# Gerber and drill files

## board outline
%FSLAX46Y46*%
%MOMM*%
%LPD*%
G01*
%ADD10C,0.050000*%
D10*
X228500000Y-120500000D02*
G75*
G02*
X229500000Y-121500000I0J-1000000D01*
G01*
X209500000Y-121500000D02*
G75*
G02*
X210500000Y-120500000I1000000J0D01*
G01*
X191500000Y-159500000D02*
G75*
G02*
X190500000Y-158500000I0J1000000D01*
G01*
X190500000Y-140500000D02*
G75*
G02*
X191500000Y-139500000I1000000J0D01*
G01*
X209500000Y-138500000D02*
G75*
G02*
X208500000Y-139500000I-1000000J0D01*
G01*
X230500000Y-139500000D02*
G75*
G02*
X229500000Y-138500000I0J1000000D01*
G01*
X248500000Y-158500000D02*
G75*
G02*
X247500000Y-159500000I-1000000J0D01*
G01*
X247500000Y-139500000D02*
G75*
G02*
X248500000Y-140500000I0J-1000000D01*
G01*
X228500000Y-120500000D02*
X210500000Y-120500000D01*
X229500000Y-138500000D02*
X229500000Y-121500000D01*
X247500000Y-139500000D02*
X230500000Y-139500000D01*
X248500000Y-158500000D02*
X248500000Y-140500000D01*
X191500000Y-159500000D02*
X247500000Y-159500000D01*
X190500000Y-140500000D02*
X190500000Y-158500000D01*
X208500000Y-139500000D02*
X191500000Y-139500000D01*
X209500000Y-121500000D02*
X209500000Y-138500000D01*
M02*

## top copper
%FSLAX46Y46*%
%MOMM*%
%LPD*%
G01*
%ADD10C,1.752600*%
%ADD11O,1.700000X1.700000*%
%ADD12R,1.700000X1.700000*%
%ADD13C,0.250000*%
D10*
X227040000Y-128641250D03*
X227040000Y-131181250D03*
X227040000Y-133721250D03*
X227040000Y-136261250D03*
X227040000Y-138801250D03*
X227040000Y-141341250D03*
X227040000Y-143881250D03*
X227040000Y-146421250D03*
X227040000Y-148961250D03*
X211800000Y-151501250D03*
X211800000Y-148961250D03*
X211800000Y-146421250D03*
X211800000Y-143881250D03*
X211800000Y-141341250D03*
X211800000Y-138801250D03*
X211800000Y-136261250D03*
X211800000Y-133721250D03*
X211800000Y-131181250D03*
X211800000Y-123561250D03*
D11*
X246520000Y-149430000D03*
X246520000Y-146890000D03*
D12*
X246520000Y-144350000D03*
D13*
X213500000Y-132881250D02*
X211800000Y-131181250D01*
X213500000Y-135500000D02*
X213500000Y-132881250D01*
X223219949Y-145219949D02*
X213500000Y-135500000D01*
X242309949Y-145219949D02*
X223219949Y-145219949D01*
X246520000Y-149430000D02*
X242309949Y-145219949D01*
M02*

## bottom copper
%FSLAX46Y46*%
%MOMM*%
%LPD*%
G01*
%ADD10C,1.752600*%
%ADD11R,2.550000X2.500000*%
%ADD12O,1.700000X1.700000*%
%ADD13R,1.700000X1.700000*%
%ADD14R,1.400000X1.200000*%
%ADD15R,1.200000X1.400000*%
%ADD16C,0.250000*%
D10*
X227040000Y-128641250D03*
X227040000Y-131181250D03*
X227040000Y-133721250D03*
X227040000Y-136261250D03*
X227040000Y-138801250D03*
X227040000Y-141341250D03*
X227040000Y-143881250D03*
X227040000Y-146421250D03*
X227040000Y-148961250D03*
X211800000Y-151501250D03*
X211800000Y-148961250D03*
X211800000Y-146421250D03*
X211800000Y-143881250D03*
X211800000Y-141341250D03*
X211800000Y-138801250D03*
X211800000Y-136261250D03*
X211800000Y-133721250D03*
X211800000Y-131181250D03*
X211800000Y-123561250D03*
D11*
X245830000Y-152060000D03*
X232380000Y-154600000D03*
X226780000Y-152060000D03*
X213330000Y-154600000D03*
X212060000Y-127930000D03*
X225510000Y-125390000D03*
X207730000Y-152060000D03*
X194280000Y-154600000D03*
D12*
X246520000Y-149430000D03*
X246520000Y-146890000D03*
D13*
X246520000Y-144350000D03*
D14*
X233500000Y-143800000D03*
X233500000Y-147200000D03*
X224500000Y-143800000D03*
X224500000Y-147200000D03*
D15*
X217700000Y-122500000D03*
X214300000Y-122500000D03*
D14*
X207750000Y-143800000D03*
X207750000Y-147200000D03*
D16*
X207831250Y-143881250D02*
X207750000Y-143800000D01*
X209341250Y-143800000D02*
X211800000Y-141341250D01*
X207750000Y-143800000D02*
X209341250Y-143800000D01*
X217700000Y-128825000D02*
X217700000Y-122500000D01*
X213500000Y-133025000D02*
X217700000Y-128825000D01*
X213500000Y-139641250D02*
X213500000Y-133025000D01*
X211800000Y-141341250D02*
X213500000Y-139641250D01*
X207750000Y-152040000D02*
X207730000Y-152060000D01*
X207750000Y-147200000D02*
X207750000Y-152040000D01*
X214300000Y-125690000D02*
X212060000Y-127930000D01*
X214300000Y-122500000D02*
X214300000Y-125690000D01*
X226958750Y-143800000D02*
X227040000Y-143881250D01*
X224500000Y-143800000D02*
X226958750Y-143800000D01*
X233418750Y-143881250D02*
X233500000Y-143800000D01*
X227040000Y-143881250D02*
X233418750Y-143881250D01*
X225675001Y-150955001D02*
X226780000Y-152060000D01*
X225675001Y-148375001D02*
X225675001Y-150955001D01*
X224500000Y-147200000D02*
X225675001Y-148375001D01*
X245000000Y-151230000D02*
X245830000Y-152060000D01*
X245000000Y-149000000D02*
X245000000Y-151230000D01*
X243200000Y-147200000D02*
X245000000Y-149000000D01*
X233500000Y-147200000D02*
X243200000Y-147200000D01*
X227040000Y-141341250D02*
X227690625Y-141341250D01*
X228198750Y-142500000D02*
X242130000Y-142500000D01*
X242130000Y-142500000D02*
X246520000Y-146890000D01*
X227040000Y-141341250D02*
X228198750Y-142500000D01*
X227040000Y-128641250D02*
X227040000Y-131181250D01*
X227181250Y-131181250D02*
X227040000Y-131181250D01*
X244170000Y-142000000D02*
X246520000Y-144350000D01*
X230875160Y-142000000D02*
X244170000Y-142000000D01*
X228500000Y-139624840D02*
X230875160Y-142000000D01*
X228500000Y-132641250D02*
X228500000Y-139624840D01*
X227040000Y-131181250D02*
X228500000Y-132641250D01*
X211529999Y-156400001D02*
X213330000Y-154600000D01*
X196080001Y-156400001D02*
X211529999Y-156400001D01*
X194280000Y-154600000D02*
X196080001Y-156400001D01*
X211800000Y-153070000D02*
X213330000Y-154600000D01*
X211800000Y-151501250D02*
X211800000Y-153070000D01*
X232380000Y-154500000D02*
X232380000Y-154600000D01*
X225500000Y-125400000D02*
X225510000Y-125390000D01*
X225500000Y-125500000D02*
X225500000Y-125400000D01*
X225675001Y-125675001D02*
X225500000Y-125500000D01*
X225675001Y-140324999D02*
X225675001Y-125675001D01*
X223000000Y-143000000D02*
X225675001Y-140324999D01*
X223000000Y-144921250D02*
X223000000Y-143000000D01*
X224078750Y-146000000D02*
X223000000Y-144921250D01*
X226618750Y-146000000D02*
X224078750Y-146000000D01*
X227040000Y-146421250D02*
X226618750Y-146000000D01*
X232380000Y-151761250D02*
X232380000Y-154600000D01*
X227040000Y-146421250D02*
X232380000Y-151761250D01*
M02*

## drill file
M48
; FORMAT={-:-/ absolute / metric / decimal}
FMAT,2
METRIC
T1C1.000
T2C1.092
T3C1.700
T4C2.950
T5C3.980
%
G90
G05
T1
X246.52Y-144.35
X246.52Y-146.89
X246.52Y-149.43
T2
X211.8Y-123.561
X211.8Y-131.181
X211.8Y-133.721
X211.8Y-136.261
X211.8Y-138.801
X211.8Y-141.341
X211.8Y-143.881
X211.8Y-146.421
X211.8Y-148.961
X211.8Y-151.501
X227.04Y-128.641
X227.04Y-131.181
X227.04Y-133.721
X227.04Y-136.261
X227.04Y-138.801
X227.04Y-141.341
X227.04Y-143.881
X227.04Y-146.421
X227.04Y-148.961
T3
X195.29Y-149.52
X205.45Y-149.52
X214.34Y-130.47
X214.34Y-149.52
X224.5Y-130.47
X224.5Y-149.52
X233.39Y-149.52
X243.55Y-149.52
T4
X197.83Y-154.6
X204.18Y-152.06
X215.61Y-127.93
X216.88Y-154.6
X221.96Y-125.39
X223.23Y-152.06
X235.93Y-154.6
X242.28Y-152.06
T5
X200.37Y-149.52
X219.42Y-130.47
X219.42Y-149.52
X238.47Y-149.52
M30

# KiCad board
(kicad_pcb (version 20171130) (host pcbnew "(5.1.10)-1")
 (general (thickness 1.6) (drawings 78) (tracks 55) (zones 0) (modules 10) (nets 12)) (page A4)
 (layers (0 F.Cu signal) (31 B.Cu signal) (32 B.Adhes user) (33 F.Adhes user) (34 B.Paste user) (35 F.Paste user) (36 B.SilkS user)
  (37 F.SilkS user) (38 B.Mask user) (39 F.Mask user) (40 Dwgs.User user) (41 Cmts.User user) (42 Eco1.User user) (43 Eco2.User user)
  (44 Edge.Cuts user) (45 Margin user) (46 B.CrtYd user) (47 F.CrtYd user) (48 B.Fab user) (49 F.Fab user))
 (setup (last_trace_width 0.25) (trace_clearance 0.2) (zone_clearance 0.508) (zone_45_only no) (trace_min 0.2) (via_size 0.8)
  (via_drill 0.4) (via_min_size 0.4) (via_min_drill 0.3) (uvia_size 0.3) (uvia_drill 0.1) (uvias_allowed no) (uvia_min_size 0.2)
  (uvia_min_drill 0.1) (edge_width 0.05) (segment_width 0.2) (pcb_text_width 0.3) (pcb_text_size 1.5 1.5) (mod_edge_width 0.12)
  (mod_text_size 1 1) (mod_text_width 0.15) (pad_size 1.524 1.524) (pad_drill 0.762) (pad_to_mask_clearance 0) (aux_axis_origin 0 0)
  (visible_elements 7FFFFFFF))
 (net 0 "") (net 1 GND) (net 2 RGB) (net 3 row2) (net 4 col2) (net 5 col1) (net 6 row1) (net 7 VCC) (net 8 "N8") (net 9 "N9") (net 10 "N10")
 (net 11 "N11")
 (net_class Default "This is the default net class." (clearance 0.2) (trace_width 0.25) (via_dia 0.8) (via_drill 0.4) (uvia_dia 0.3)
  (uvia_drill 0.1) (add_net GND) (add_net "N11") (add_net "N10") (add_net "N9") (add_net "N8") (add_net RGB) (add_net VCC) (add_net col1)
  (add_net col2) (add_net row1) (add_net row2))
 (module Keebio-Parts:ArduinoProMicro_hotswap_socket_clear (layer B.Cu) (at 219.42 137.53125 270)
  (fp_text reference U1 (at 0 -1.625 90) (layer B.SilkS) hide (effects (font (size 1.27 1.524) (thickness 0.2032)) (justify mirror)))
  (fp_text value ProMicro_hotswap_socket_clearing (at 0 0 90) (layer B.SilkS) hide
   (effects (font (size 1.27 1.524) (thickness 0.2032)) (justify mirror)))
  (pad 3 thru_hole circle (at -8.89 -7.62 270) (size 1.7526 1.7526) (drill 1.0922) (layers *.Cu *.SilkS *.Mask) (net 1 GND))
  (pad 4 thru_hole circle (at -6.35 -7.62 270) (size 1.7526 1.7526) (drill 1.0922) (layers *.Cu *.SilkS *.Mask) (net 1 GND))
  (pad 5 thru_hole circle (at -3.81 -7.62 270) (size 1.7526 1.7526) (drill 1.0922) (layers *.Cu *.SilkS *.Mask))
  (pad 6 thru_hole circle (at -1.27 -7.62 270) (size 1.7526 1.7526) (drill 1.0922) (layers *.Cu *.SilkS *.Mask))
  (pad 7 thru_hole circle (at 1.27 -7.62 270) (size 1.7526 1.7526) (drill 1.0922) (layers *.Cu *.SilkS *.Mask))
  (pad 8 thru_hole circle (at 3.81 -7.62 270) (size 1.7526 1.7526) (drill 1.0922) (layers *.Cu *.SilkS *.Mask) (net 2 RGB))
  (pad 9 thru_hole circle (at 6.35 -7.62 270) (size 1.7526 1.7526) (drill 1.0922) (layers *.Cu *.SilkS *.Mask) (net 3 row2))
  (pad 10 thru_hole circle (at 8.89 -7.62 270) (size 1.7526 1.7526) (drill 1.0922) (layers *.Cu *.SilkS *.Mask) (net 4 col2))
  (pad 11 thru_hole circle (at 11.43 -7.62 270) (size 1.7526 1.7526) (drill 1.0922) (layers *.Cu *.SilkS *.Mask))
  (pad 13 thru_hole circle (at 13.97 7.62 270) (size 1.7526 1.7526) (drill 1.0922) (layers *.Cu *.SilkS *.Mask) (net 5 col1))
  (pad 14 thru_hole circle (at 11.43 7.62 270) (size 1.7526 1.7526) (drill 1.0922) (layers *.Cu *.SilkS *.Mask))
  (pad 15 thru_hole circle (at 8.89 7.62 270) (size 1.7526 1.7526) (drill 1.0922) (layers *.Cu *.SilkS *.Mask))
  (pad 16 thru_hole circle (at 6.35 7.62 270) (size 1.7526 1.7526) (drill 1.0922) (layers *.Cu *.SilkS *.Mask))
  (pad 17 thru_hole circle (at 3.81 7.62 270) (size 1.7526 1.7526) (drill 1.0922) (layers *.Cu *.SilkS *.Mask) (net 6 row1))
  (pad 18 thru_hole circle (at 1.27 7.62 270) (size 1.7526 1.7526) (drill 1.0922) (layers *.Cu *.SilkS *.Mask))
  (pad 19 thru_hole circle (at -1.27 7.62 270) (size 1.7526 1.7526) (drill 1.0922) (layers *.Cu *.SilkS *.Mask))
  (pad 20 thru_hole circle (at -3.81 7.62 270) (size 1.7526 1.7526) (drill 1.0922) (layers *.Cu *.SilkS *.Mask))
  (pad 21 thru_hole circle (at -6.35 7.62 270) (size 1.7526 1.7526) (drill 1.0922) (layers *.Cu *.SilkS *.Mask) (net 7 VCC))
  (pad 24 thru_hole circle (at -13.97 7.62 270) (size 1.7526 1.7526) (drill 1.0922) (layers *.Cu *.SilkS *.Mask)))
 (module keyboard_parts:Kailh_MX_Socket (layer F.Cu) (at 238.47 149.52)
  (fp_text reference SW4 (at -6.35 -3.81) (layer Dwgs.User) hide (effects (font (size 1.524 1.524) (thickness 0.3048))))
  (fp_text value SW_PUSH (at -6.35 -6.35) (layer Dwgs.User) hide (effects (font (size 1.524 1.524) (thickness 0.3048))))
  (pad 1 smd rect (at 7.36 2.54) (size 2.55 2.5) (layers B.Cu B.Paste B.Mask) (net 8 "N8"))
  (pad "" np_thru_hole circle (at 0 0) (size 3.98018 3.98018) (drill 3.98018) (layers *.Cu *.Mask))
  (pad "" np_thru_hole circle (at -2.54 5.08) (size 2.95 2.95) (drill 2.95) (layers *.Cu *.Mask))
  (pad "" np_thru_hole circle (at 3.81 2.54) (size 2.95 2.95) (drill 2.95) (layers *.Cu *.Mask))
  (pad 2 smd rect (at -6.09 5.08) (size 2.55 2.5) (layers B.Cu B.Paste B.Mask) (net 4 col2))
  (pad "" np_thru_hole circle (at -5.08 0) (size 1.7 1.7) (drill 1.7) (layers *.Cu *.Mask))
  (pad "" np_thru_hole circle (at 5.08 0) (size 1.7 1.7) (drill 1.7) (layers *.Cu *.Mask)))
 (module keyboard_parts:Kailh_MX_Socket (layer F.Cu) (at 219.42 149.52)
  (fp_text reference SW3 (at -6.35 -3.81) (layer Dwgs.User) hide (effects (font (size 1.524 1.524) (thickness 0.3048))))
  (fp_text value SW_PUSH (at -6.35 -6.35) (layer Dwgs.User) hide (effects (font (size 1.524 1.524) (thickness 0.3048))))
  (pad 1 smd rect (at 7.36 2.54) (size 2.55 2.5) (layers B.Cu B.Paste B.Mask) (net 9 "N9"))
  (pad "" np_thru_hole circle (at 0 0) (size 3.98018 3.98018) (drill 3.98018) (layers *.Cu *.Mask))
  (pad "" np_thru_hole circle (at -2.54 5.08) (size 2.95 2.95) (drill 2.95) (layers *.Cu *.Mask))
  (pad "" np_thru_hole circle (at 3.81 2.54) (size 2.95 2.95) (drill 2.95) (layers *.Cu *.Mask))
  (pad 2 smd rect (at -6.09 5.08) (size 2.55 2.5) (layers B.Cu B.Paste B.Mask) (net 5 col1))
  (pad "" np_thru_hole circle (at -5.08 0) (size 1.7 1.7) (drill 1.7) (layers *.Cu *.Mask))
  (pad "" np_thru_hole circle (at 5.08 0) (size 1.7 1.7) (drill 1.7) (layers *.Cu *.Mask)))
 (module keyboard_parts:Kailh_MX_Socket (layer F.Cu) (at 219.42 130.47 180)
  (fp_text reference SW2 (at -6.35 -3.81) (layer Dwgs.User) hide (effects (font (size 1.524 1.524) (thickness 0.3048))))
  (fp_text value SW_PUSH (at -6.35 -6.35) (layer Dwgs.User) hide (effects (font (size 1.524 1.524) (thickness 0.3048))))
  (pad 1 smd rect (at 7.36 2.54 180) (size 2.55 2.5) (layers B.Cu B.Paste B.Mask) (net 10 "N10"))
  (pad "" np_thru_hole circle (at 0 0 180) (size 3.98018 3.98018) (drill 3.98018) (layers *.Cu *.Mask))
  (pad "" np_thru_hole circle (at -2.54 5.08 180) (size 2.95 2.95) (drill 2.95) (layers *.Cu *.Mask))
  (pad "" np_thru_hole circle (at 3.81 2.54 180) (size 2.95 2.95) (drill 2.95) (layers *.Cu *.Mask))
  (pad 2 smd rect (at -6.09 5.08 180) (size 2.55 2.5) (layers B.Cu B.Paste B.Mask) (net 4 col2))
  (pad "" np_thru_hole circle (at -5.08 0 180) (size 1.7 1.7) (drill 1.7) (layers *.Cu *.Mask))
  (pad "" np_thru_hole circle (at 5.08 0 180) (size 1.7 1.7) (drill 1.7) (layers *.Cu *.Mask)))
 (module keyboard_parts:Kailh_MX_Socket (layer F.Cu) (at 200.37 149.52)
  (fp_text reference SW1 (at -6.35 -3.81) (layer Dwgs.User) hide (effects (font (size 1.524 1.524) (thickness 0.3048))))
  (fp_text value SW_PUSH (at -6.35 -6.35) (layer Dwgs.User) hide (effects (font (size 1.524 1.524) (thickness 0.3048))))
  (pad 1 smd rect (at 7.36 2.54) (size 2.55 2.5) (layers B.Cu B.Paste B.Mask) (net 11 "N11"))
  (pad "" np_thru_hole circle (at 0 0) (size 3.98018 3.98018) (drill 3.98018) (layers *.Cu *.Mask))
  (pad "" np_thru_hole circle (at -2.54 5.08) (size 2.95 2.95) (drill 2.95) (layers *.Cu *.Mask))
  (pad "" np_thru_hole circle (at 3.81 2.54) (size 2.95 2.95) (drill 2.95) (layers *.Cu *.Mask))
  (pad 2 smd rect (at -6.09 5.08) (size 2.55 2.5) (layers B.Cu B.Paste B.Mask) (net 5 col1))
  (pad "" np_thru_hole circle (at -5.08 0) (size 1.7 1.7) (drill 1.7) (layers *.Cu *.Mask))
  (pad "" np_thru_hole circle (at 5.08 0) (size 1.7 1.7) (drill 1.7) (layers *.Cu *.Mask)))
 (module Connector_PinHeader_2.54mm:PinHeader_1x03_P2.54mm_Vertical (layer F.Cu) (at 246.52 144.35)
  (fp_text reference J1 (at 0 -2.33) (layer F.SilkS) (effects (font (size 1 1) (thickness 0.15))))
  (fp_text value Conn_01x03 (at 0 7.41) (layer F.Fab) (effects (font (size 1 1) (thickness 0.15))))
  (pad 3 thru_hole oval (at 0 5.08) (size 1.7 1.7) (drill 1) (layers *.Cu *.Mask) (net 7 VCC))
  (pad 2 thru_hole oval (at 0 2.54) (size 1.7 1.7) (drill 1) (layers *.Cu *.Mask) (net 2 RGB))
  (pad 1 thru_hole rect (at 0 0) (size 1.7 1.7) (drill 1) (layers *.Cu *.Mask) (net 1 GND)))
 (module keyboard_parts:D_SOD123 (layer B.Cu) (at 233.5 145.5 270)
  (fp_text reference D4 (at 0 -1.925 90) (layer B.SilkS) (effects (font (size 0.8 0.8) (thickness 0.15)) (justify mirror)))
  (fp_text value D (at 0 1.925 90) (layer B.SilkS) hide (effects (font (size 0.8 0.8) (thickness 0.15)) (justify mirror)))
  (pad 1 smd rect (at -1.7 0 270) (size 1.2 1.4) (layers B.Cu B.Paste B.Mask) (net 3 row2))
  (pad 2 smd rect (at 1.7 0 270) (size 1.2 1.4) (layers B.Cu B.Paste B.Mask) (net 8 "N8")))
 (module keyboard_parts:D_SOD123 (layer B.Cu) (at 224.5 145.5 270)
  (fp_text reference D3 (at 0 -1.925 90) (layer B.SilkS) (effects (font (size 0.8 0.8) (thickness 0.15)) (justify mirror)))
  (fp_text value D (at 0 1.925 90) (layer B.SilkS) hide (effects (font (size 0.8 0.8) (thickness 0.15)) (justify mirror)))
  (pad 1 smd rect (at -1.7 0 270) (size 1.2 1.4) (layers B.Cu B.Paste B.Mask) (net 3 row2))
  (pad 2 smd rect (at 1.7 0 270) (size 1.2 1.4) (layers B.Cu B.Paste B.Mask) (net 9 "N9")))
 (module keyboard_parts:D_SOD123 (layer B.Cu) (at 216 122.5 180)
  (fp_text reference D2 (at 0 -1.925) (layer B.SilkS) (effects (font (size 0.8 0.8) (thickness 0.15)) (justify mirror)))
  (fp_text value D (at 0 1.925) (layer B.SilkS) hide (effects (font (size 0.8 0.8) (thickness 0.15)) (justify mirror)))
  (pad 1 smd rect (at -1.7 0 180) (size 1.2 1.4) (layers B.Cu B.Paste B.Mask) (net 6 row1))
  (pad 2 smd rect (at 1.7 0 180) (size 1.2 1.4) (layers B.Cu B.Paste B.Mask) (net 10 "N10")))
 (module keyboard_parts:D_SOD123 (layer B.Cu) (at 207.75 145.5 270)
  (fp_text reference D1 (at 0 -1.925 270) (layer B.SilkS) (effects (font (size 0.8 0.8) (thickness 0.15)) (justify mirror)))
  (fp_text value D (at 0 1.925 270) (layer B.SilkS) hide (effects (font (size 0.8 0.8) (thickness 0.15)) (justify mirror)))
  (pad 1 smd rect (at -1.7 0 270) (size 1.2 1.4) (layers B.Cu B.Paste B.Mask) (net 6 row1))
  (pad 2 smd rect (at 1.7 0 270) (size 1.2 1.4) (layers B.Cu B.Paste B.Mask) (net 11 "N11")))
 (gr_arc (start 228.5 121.5) (end 229.5 121.5) (angle -90) (layer Edge.Cuts) (width 0.05))
 (gr_arc (start 210.5 121.5) (end 210.5 120.5) (angle -90) (layer Edge.Cuts) (width 0.05))
 (gr_arc (start 191.5 158.5) (end 190.5 158.5) (angle -90) (layer Edge.Cuts) (width 0.05))
 (gr_arc (start 191.5 140.5) (end 191.5 139.5) (angle -90) (layer Edge.Cuts) (width 0.05))
 (gr_arc (start 208.5 138.5) (end 208.5 139.5) (angle -90) (layer Edge.Cuts) (width 0.05))
 (gr_arc (start 230.5 138.5) (end 229.5 138.5) (angle -90) (layer Edge.Cuts) (width 0.05))
 (gr_arc (start 247.5 158.5) (end 247.5 159.5) (angle -90) (layer Edge.Cuts) (width 0.05))
 (gr_arc (start 247.5 140.5) (end 248.5 140.5) (angle -90) (layer Edge.Cuts) (width 0.05))
 (gr_line (start 228.5 120.5) (end 210.5 120.5) (layer Edge.Cuts) (width 0.05))
 (gr_line (start 229.5 138.5) (end 229.5 121.5) (layer Edge.Cuts) (width 0.05))
 (gr_line (start 247.5 139.5) (end 230.5 139.5) (layer Edge.Cuts) (width 0.05))
 (gr_line (start 248.5 158.5) (end 248.5 140.5) (layer Edge.Cuts) (width 0.05))
 (gr_line (start 191.5 159.5) (end 247.5 159.5) (layer Edge.Cuts) (width 0.05))
 (gr_line (start 190.5 140.5) (end 190.5 158.5) (layer Edge.Cuts) (width 0.05))
 (gr_line (start 208.5 139.5) (end 191.5 139.5) (layer Edge.Cuts) (width 0.05))
 (gr_line (start 209.5 121.5) (end 209.5 138.5) (layer Edge.Cuts) (width 0.05))
 (segment (start 207.83125 143.88125) (end 207.75 143.8) (width 0.25) (layer B.Cu) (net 6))
 (segment (start 209.34125 143.8) (end 211.8 141.34125) (width 0.25) (layer B.Cu) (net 6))
 (segment (start 207.75 143.8) (end 209.34125 143.8) (width 0.25) (layer B.Cu) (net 6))
 (segment (start 217.7 128.825) (end 217.7 122.5) (width 0.25) (layer B.Cu) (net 6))
 (segment (start 213.5 133.025) (end 217.7 128.825) (width 0.25) (layer B.Cu) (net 6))
 (segment (start 213.5 139.64125) (end 213.5 133.025) (width 0.25) (layer B.Cu) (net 6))
 (segment (start 211.8 141.34125) (end 213.5 139.64125) (width 0.25) (layer B.Cu) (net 6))
 (segment (start 207.75 152.04) (end 207.73 152.06) (width 0.25) (layer B.Cu) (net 11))
 (segment (start 207.75 147.2) (end 207.75 152.04) (width 0.25) (layer B.Cu) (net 11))
 (segment (start 214.3 125.69) (end 212.06 127.93) (width 0.25) (layer B.Cu) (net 10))
 (segment (start 214.3 122.5) (end 214.3 125.69) (width 0.25) (layer B.Cu) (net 10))
 (segment (start 226.95875 143.8) (end 227.04 143.88125) (width 0.25) (layer B.Cu) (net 3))
 (segment (start 224.5 143.8) (end 226.95875 143.8) (width 0.25) (layer B.Cu) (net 3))
 (segment (start 233.41875 143.88125) (end 233.5 143.8) (width 0.25) (layer B.Cu) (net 3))
 (segment (start 227.04 143.88125) (end 233.41875 143.88125) (width 0.25) (layer B.Cu) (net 3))
 (segment (start 225.675001 150.955001) (end 226.78 152.06) (width 0.25) (layer B.Cu) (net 9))
 (segment (start 225.675001 148.375001) (end 225.675001 150.955001) (width 0.25) (layer B.Cu) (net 9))
 (segment (start 224.5 147.2) (end 225.675001 148.375001) (width 0.25) (layer B.Cu) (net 9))
 (segment (start 245 151.23) (end 245.83 152.06) (width 0.25) (layer B.Cu) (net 8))
 (segment (start 245 149) (end 245 151.23) (width 0.25) (layer B.Cu) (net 8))
 (segment (start 243.2 147.2) (end 245 149) (width 0.25) (layer B.Cu) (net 8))
 (segment (start 233.5 147.2) (end 243.2 147.2) (width 0.25) (layer B.Cu) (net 8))
 (segment (start 213.5 132.88125) (end 211.8 131.18125) (width 0.25) (layer F.Cu) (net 7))
 (segment (start 213.5 135.5) (end 213.5 132.88125) (width 0.25) (layer F.Cu) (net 7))
 (segment (start 223.219949 145.219949) (end 213.5 135.5) (width 0.25) (layer F.Cu) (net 7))
 (segment (start 242.309949 145.219949) (end 223.219949 145.219949) (width 0.25) (layer F.Cu) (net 7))
 (segment (start 246.52 149.43) (end 242.309949 145.219949) (width 0.25) (layer F.Cu) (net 7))
 (segment (start 227.04 141.34125) (end 227.690625 141.34125) (width 0.25) (layer B.Cu) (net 2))
 (segment (start 228.19875 142.5) (end 242.13 142.5) (width 0.25) (layer B.Cu) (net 2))
 (segment (start 242.13 142.5) (end 246.52 146.89) (width 0.25) (layer B.Cu) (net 2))
 (segment (start 227.04 141.34125) (end 228.19875 142.5) (width 0.25) (layer B.Cu) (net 2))
 (segment (start 227.04 128.64125) (end 227.04 131.18125) (width 0.25) (layer B.Cu) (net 1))
 (segment (start 227.18125 131.18125) (end 227.04 131.18125) (width 0.25) (layer B.Cu) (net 1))
 (segment (start 244.17 142) (end 246.52 144.35) (width 0.25) (layer B.Cu) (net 1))
 (segment (start 230.87516 142) (end 244.17 142) (width 0.25) (layer B.Cu) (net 1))
 (segment (start 228.5 139.62484) (end 230.87516 142) (width 0.25) (layer B.Cu) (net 1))
 (segment (start 228.5 132.64125) (end 228.5 139.62484) (width 0.25) (layer B.Cu) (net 1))
 (segment (start 227.04 131.18125) (end 228.5 132.64125) (width 0.25) (layer B.Cu) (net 1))
 (segment (start 211.529999 156.400001) (end 213.33 154.6) (width 0.25) (layer B.Cu) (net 5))
 (segment (start 196.080001 156.400001) (end 211.529999 156.400001) (width 0.25) (layer B.Cu) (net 5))
 (segment (start 194.28 154.6) (end 196.080001 156.400001) (width 0.25) (layer B.Cu) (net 5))
 (segment (start 211.8 153.07) (end 213.33 154.6) (width 0.25) (layer B.Cu) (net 5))
 (segment (start 211.8 151.50125) (end 211.8 153.07) (width 0.25) (layer B.Cu) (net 5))
 (segment (start 232.38 154.5) (end 232.38 154.6) (width 0.25) (layer B.Cu) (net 4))
 (segment (start 225.5 125.4) (end 225.51 125.39) (width 0.25) (layer B.Cu) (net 4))
 (segment (start 225.5 125.5) (end 225.5 125.4) (width 0.25) (layer B.Cu) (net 4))
 (segment (start 225.675001 125.675001) (end 225.5 125.5) (width 0.25) (layer B.Cu) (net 4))
 (segment (start 225.675001 140.324999) (end 225.675001 125.675001) (width 0.25) (layer B.Cu) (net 4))
 (segment (start 223 143) (end 225.675001 140.324999) (width 0.25) (layer B.Cu) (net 4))
 (segment (start 223 144.92125) (end 223 143) (width 0.25) (layer B.Cu) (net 4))
 (segment (start 224.07875 146) (end 223 144.92125) (width 0.25) (layer B.Cu) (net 4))
 (segment (start 226.61875 146) (end 224.07875 146) (width 0.25) (layer B.Cu) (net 4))
 (segment (start 227.04 146.42125) (end 226.61875 146) (width 0.25) (layer B.Cu) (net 4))
 (segment (start 232.38 151.76125) (end 232.38 154.6) (width 0.25) (layer B.Cu) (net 4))
 (segment (start 227.04 146.42125) (end 232.38 151.76125) (width 0.25) (layer B.Cu) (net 4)))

